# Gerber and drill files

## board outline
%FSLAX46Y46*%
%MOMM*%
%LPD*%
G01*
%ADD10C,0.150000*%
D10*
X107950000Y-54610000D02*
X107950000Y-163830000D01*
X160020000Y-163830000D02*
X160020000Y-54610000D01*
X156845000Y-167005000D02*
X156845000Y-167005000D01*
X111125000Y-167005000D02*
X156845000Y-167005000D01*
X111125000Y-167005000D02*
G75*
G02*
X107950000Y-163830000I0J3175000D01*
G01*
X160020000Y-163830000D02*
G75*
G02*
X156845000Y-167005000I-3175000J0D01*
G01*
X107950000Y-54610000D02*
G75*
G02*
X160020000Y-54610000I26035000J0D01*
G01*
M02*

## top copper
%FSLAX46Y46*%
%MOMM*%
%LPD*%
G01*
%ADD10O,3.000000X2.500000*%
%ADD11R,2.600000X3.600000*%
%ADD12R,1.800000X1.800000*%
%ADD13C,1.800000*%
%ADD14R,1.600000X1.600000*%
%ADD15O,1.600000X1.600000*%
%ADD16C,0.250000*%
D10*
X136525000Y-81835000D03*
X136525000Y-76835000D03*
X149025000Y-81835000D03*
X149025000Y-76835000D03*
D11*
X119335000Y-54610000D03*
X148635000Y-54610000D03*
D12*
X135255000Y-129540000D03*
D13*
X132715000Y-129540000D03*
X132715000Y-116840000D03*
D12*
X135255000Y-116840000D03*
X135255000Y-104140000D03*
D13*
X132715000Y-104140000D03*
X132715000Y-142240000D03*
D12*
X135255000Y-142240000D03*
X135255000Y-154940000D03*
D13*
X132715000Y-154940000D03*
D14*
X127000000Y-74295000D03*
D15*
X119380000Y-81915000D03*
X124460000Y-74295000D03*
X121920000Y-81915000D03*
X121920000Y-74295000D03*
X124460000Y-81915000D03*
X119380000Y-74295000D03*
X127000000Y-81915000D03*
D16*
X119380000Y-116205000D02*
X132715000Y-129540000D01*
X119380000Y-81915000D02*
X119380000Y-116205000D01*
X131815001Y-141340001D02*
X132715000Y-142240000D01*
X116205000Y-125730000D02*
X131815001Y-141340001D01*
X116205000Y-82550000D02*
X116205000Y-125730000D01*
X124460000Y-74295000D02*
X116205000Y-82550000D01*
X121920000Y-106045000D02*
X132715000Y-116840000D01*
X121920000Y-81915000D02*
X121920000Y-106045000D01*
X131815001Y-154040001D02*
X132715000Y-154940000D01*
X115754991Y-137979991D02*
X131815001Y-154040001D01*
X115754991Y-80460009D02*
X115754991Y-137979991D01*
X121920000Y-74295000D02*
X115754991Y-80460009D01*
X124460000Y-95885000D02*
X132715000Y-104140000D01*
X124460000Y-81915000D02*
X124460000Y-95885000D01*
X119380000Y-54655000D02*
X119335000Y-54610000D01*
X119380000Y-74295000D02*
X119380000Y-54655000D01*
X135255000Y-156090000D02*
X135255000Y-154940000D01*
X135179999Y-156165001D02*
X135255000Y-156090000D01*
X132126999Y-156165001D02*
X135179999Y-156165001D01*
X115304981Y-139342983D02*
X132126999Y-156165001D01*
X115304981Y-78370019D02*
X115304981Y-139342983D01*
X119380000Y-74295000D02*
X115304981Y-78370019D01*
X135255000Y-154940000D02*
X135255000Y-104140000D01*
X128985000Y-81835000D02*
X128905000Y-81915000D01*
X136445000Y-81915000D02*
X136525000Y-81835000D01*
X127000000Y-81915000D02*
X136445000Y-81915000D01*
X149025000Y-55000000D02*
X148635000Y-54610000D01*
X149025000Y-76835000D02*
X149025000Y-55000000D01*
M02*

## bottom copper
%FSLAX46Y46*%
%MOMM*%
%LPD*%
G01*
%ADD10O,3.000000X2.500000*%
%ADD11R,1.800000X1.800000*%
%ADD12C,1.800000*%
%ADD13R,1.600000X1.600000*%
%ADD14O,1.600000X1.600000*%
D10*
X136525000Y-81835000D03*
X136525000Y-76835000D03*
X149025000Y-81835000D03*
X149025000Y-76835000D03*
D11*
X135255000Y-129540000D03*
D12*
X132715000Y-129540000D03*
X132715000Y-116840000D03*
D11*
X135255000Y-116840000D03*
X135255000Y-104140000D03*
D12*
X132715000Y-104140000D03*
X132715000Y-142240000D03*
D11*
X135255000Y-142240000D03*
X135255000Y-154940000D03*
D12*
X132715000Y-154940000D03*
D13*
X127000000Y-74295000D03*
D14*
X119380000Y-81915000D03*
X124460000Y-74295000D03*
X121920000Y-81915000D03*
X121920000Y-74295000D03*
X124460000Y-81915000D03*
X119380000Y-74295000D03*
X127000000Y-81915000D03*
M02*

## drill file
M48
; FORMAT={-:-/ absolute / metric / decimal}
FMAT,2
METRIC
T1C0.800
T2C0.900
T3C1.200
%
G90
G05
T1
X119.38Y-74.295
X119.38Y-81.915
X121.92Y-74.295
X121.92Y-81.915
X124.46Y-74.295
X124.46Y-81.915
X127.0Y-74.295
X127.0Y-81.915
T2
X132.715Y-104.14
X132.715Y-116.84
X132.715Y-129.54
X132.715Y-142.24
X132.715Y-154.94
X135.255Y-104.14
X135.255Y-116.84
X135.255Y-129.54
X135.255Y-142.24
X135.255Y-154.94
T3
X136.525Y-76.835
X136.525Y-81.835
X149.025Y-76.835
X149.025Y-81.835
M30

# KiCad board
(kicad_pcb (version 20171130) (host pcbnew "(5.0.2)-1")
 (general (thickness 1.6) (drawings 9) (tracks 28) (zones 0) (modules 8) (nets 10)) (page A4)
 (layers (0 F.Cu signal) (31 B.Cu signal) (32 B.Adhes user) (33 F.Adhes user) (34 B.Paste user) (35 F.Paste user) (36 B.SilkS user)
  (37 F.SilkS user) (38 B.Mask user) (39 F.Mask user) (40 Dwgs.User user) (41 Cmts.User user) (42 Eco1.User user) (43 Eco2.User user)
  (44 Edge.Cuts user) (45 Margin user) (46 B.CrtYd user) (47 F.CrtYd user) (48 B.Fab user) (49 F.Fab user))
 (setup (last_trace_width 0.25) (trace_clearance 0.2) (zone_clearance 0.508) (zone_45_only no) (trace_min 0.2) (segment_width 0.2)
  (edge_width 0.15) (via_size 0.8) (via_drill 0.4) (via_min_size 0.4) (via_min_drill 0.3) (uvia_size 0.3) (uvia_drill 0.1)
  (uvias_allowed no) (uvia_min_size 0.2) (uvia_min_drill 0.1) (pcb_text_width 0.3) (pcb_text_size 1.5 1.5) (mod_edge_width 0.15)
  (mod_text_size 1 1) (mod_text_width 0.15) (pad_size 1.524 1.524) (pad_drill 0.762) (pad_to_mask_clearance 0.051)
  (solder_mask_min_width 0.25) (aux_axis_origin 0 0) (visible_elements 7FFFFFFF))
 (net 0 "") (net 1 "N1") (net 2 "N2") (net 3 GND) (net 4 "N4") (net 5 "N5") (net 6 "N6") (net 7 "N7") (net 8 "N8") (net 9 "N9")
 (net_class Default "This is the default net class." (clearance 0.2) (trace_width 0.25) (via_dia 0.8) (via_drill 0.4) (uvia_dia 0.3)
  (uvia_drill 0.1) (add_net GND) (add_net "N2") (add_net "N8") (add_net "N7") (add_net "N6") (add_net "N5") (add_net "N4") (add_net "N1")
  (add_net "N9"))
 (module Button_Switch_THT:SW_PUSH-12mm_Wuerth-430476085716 (layer F.Cu) (at 136.525 76.835)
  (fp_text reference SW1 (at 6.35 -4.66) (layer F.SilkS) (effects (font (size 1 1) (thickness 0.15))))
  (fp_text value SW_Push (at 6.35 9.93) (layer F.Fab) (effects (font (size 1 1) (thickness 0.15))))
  (pad 2 thru_hole oval (at 0 5) (size 3 2.5) (drill 1.2) (layers *.Cu *.Mask) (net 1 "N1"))
  (pad 1 thru_hole oval (at 0 0) (size 3 2.5) (drill 1.2) (layers *.Cu *.Mask) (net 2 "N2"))
  (pad 2 thru_hole oval (at 12.5 5) (size 3 2.5) (drill 1.2) (layers *.Cu *.Mask) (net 1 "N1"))
  (pad 1 thru_hole oval (at 12.5 0) (size 3 2.5) (drill 1.2) (layers *.Cu *.Mask) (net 2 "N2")))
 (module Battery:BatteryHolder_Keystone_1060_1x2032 (layer F.Cu) (at 133.985 54.61 180)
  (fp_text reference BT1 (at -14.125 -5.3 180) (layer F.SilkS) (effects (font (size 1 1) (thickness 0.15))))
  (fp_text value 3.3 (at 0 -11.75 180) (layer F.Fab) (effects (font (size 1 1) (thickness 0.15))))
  (pad 2 smd rect (at 14.65 0) (size 2.6 3.6) (layers F.Cu F.Paste F.Mask) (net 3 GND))
  (pad 1 smd rect (at -14.65 0) (size 2.6 3.6) (layers F.Cu F.Paste F.Mask) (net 2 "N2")))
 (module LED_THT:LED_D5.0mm (layer F.Cu) (at 135.255 129.54 180)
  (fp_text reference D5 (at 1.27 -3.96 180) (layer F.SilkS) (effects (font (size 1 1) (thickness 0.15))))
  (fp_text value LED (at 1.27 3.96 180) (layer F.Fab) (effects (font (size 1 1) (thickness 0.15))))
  (pad 1 thru_hole rect (at 0 0 180) (size 1.8 1.8) (drill 0.9) (layers *.Cu *.Mask) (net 3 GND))
  (pad 2 thru_hole circle (at 2.54 0 180) (size 1.8 1.8) (drill 0.9) (layers *.Cu *.Mask) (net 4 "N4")))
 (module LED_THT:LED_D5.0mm (layer F.Cu) (at 135.255 116.84 180)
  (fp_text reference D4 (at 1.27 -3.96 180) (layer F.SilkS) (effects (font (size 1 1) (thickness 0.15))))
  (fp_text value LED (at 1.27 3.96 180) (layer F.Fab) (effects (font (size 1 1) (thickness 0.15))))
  (pad 2 thru_hole circle (at 2.54 0 180) (size 1.8 1.8) (drill 0.9) (layers *.Cu *.Mask) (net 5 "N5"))
  (pad 1 thru_hole rect (at 0 0 180) (size 1.8 1.8) (drill 0.9) (layers *.Cu *.Mask) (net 3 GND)))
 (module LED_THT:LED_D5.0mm (layer F.Cu) (at 135.255 104.14 180)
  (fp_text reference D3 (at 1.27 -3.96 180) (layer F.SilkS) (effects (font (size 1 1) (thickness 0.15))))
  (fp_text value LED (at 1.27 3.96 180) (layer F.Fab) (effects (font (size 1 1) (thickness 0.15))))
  (pad 1 thru_hole rect (at 0 0 180) (size 1.8 1.8) (drill 0.9) (layers *.Cu *.Mask) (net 3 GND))
  (pad 2 thru_hole circle (at 2.54 0 180) (size 1.8 1.8) (drill 0.9) (layers *.Cu *.Mask) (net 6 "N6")))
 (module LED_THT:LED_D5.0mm (layer F.Cu) (at 135.255 142.24 180)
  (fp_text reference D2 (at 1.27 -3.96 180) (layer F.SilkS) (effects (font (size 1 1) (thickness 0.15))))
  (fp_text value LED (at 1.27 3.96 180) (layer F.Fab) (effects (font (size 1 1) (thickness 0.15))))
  (pad 2 thru_hole circle (at 2.54 0 180) (size 1.8 1.8) (drill 0.9) (layers *.Cu *.Mask) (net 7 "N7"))
  (pad 1 thru_hole rect (at 0 0 180) (size 1.8 1.8) (drill 0.9) (layers *.Cu *.Mask) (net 3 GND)))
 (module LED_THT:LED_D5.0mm (layer F.Cu) (at 135.255 154.94 180)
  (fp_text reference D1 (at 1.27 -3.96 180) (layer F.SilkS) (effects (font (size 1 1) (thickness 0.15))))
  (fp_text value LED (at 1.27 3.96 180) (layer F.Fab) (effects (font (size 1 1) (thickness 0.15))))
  (pad 1 thru_hole rect (at 0 0 180) (size 1.8 1.8) (drill 0.9) (layers *.Cu *.Mask) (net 3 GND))
  (pad 2 thru_hole circle (at 2.54 0 180) (size 1.8 1.8) (drill 0.9) (layers *.Cu *.Mask) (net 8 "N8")))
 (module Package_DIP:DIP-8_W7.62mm (layer F.Cu) (at 127 74.295 270)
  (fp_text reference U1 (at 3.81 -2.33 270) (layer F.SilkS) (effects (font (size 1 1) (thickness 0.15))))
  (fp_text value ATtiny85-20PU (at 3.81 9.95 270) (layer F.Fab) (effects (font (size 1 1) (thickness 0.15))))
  (pad 1 thru_hole rect (at 0 0 270) (size 1.6 1.6) (drill 0.8) (layers *.Cu *.Mask) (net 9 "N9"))
  (pad 5 thru_hole oval (at 7.62 7.62 270) (size 1.6 1.6) (drill 0.8) (layers *.Cu *.Mask) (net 4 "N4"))
  (pad 2 thru_hole oval (at 0 2.54 270) (size 1.6 1.6) (drill 0.8) (layers *.Cu *.Mask) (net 7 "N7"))
  (pad 6 thru_hole oval (at 7.62 5.08 270) (size 1.6 1.6) (drill 0.8) (layers *.Cu *.Mask) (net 5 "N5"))
  (pad 3 thru_hole oval (at 0 5.08 270) (size 1.6 1.6) (drill 0.8) (layers *.Cu *.Mask) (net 8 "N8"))
  (pad 7 thru_hole oval (at 7.62 2.54 270) (size 1.6 1.6) (drill 0.8) (layers *.Cu *.Mask) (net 6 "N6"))
  (pad 4 thru_hole oval (at 0 7.62 270) (size 1.6 1.6) (drill 0.8) (layers *.Cu *.Mask) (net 3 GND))
  (pad 8 thru_hole oval (at 7.62 0 270) (size 1.6 1.6) (drill 0.8) (layers *.Cu *.Mask) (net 1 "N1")))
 (gr_line (start 107.95 54.61) (end 107.95 163.83) (layer Edge.Cuts) (width 0.15))
 (gr_line (start 160.02 163.83) (end 160.02 54.61) (layer Edge.Cuts) (width 0.15))
 (gr_line (start 156.845 167.005) (end 156.845 167.005) (layer Edge.Cuts) (width 0.15))
 (gr_line (start 111.125 167.005) (end 156.845 167.005) (layer Edge.Cuts) (width 0.15))
 (gr_arc (start 111.125 163.83) (end 107.95 163.83) (angle -90) (layer Edge.Cuts) (width 0.15))
 (gr_arc (start 156.845 163.83) (end 156.845 167.005) (angle -90) (layer Edge.Cuts) (width 0.15))
 (gr_arc (start 133.985 54.61) (end 160.02 54.61) (angle -180) (layer Edge.Cuts) (width 0.15))
 (segment (start 119.38 116.205) (end 132.715 129.54) (width 0.25) (layer F.Cu) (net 4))
 (segment (start 119.38 81.915) (end 119.38 116.205) (width 0.25) (layer F.Cu) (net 4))
 (segment (start 131.815001 141.340001) (end 132.715 142.24) (width 0.25) (layer F.Cu) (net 7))
 (segment (start 116.205 125.73) (end 131.815001 141.340001) (width 0.25) (layer F.Cu) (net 7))
 (segment (start 116.205 82.55) (end 116.205 125.73) (width 0.25) (layer F.Cu) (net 7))
 (segment (start 124.46 74.295) (end 116.205 82.55) (width 0.25) (layer F.Cu) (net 7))
 (segment (start 121.92 106.045) (end 132.715 116.84) (width 0.25) (layer F.Cu) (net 5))
 (segment (start 121.92 81.915) (end 121.92 106.045) (width 0.25) (layer F.Cu) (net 5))
 (segment (start 131.815001 154.040001) (end 132.715 154.94) (width 0.25) (layer F.Cu) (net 8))
 (segment (start 115.754991 137.979991) (end 131.815001 154.040001) (width 0.25) (layer F.Cu) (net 8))
 (segment (start 115.754991 80.460009) (end 115.754991 137.979991) (width 0.25) (layer F.Cu) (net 8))
 (segment (start 121.92 74.295) (end 115.754991 80.460009) (width 0.25) (layer F.Cu) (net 8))
 (segment (start 124.46 95.885) (end 132.715 104.14) (width 0.25) (layer F.Cu) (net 6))
 (segment (start 124.46 81.915) (end 124.46 95.885) (width 0.25) (layer F.Cu) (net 6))
 (segment (start 119.38 54.655) (end 119.335 54.61) (width 0.25) (layer F.Cu) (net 3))
 (segment (start 119.38 74.295) (end 119.38 54.655) (width 0.25) (layer F.Cu) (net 3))
 (segment (start 135.255 156.09) (end 135.255 154.94) (width 0.25) (layer F.Cu) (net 3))
 (segment (start 135.179999 156.165001) (end 135.255 156.09) (width 0.25) (layer F.Cu) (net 3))
 (segment (start 132.126999 156.165001) (end 135.179999 156.165001) (width 0.25) (layer F.Cu) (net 3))
 (segment (start 115.304981 139.342983) (end 132.126999 156.165001) (width 0.25) (layer F.Cu) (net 3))
 (segment (start 115.304981 78.370019) (end 115.304981 139.342983) (width 0.25) (layer F.Cu) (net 3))
 (segment (start 119.38 74.295) (end 115.304981 78.370019) (width 0.25) (layer F.Cu) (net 3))
 (segment (start 135.255 154.94) (end 135.255 104.14) (width 0.25) (layer F.Cu) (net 3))
 (segment (start 128.985 81.835) (end 128.905 81.915) (width 0.25) (layer F.Cu) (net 1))
 (segment (start 136.445 81.915) (end 136.525 81.835) (width 0.25) (layer F.Cu) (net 1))
 (segment (start 127 81.915) (end 136.445 81.915) (width 0.25) (layer F.Cu) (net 1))
 (segment (start 149.025 55) (end 148.635 54.61) (width 0.25) (layer F.Cu) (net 2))
 (segment (start 149.025 76.835) (end 149.025 55) (width 0.25) (layer F.Cu) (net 2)))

